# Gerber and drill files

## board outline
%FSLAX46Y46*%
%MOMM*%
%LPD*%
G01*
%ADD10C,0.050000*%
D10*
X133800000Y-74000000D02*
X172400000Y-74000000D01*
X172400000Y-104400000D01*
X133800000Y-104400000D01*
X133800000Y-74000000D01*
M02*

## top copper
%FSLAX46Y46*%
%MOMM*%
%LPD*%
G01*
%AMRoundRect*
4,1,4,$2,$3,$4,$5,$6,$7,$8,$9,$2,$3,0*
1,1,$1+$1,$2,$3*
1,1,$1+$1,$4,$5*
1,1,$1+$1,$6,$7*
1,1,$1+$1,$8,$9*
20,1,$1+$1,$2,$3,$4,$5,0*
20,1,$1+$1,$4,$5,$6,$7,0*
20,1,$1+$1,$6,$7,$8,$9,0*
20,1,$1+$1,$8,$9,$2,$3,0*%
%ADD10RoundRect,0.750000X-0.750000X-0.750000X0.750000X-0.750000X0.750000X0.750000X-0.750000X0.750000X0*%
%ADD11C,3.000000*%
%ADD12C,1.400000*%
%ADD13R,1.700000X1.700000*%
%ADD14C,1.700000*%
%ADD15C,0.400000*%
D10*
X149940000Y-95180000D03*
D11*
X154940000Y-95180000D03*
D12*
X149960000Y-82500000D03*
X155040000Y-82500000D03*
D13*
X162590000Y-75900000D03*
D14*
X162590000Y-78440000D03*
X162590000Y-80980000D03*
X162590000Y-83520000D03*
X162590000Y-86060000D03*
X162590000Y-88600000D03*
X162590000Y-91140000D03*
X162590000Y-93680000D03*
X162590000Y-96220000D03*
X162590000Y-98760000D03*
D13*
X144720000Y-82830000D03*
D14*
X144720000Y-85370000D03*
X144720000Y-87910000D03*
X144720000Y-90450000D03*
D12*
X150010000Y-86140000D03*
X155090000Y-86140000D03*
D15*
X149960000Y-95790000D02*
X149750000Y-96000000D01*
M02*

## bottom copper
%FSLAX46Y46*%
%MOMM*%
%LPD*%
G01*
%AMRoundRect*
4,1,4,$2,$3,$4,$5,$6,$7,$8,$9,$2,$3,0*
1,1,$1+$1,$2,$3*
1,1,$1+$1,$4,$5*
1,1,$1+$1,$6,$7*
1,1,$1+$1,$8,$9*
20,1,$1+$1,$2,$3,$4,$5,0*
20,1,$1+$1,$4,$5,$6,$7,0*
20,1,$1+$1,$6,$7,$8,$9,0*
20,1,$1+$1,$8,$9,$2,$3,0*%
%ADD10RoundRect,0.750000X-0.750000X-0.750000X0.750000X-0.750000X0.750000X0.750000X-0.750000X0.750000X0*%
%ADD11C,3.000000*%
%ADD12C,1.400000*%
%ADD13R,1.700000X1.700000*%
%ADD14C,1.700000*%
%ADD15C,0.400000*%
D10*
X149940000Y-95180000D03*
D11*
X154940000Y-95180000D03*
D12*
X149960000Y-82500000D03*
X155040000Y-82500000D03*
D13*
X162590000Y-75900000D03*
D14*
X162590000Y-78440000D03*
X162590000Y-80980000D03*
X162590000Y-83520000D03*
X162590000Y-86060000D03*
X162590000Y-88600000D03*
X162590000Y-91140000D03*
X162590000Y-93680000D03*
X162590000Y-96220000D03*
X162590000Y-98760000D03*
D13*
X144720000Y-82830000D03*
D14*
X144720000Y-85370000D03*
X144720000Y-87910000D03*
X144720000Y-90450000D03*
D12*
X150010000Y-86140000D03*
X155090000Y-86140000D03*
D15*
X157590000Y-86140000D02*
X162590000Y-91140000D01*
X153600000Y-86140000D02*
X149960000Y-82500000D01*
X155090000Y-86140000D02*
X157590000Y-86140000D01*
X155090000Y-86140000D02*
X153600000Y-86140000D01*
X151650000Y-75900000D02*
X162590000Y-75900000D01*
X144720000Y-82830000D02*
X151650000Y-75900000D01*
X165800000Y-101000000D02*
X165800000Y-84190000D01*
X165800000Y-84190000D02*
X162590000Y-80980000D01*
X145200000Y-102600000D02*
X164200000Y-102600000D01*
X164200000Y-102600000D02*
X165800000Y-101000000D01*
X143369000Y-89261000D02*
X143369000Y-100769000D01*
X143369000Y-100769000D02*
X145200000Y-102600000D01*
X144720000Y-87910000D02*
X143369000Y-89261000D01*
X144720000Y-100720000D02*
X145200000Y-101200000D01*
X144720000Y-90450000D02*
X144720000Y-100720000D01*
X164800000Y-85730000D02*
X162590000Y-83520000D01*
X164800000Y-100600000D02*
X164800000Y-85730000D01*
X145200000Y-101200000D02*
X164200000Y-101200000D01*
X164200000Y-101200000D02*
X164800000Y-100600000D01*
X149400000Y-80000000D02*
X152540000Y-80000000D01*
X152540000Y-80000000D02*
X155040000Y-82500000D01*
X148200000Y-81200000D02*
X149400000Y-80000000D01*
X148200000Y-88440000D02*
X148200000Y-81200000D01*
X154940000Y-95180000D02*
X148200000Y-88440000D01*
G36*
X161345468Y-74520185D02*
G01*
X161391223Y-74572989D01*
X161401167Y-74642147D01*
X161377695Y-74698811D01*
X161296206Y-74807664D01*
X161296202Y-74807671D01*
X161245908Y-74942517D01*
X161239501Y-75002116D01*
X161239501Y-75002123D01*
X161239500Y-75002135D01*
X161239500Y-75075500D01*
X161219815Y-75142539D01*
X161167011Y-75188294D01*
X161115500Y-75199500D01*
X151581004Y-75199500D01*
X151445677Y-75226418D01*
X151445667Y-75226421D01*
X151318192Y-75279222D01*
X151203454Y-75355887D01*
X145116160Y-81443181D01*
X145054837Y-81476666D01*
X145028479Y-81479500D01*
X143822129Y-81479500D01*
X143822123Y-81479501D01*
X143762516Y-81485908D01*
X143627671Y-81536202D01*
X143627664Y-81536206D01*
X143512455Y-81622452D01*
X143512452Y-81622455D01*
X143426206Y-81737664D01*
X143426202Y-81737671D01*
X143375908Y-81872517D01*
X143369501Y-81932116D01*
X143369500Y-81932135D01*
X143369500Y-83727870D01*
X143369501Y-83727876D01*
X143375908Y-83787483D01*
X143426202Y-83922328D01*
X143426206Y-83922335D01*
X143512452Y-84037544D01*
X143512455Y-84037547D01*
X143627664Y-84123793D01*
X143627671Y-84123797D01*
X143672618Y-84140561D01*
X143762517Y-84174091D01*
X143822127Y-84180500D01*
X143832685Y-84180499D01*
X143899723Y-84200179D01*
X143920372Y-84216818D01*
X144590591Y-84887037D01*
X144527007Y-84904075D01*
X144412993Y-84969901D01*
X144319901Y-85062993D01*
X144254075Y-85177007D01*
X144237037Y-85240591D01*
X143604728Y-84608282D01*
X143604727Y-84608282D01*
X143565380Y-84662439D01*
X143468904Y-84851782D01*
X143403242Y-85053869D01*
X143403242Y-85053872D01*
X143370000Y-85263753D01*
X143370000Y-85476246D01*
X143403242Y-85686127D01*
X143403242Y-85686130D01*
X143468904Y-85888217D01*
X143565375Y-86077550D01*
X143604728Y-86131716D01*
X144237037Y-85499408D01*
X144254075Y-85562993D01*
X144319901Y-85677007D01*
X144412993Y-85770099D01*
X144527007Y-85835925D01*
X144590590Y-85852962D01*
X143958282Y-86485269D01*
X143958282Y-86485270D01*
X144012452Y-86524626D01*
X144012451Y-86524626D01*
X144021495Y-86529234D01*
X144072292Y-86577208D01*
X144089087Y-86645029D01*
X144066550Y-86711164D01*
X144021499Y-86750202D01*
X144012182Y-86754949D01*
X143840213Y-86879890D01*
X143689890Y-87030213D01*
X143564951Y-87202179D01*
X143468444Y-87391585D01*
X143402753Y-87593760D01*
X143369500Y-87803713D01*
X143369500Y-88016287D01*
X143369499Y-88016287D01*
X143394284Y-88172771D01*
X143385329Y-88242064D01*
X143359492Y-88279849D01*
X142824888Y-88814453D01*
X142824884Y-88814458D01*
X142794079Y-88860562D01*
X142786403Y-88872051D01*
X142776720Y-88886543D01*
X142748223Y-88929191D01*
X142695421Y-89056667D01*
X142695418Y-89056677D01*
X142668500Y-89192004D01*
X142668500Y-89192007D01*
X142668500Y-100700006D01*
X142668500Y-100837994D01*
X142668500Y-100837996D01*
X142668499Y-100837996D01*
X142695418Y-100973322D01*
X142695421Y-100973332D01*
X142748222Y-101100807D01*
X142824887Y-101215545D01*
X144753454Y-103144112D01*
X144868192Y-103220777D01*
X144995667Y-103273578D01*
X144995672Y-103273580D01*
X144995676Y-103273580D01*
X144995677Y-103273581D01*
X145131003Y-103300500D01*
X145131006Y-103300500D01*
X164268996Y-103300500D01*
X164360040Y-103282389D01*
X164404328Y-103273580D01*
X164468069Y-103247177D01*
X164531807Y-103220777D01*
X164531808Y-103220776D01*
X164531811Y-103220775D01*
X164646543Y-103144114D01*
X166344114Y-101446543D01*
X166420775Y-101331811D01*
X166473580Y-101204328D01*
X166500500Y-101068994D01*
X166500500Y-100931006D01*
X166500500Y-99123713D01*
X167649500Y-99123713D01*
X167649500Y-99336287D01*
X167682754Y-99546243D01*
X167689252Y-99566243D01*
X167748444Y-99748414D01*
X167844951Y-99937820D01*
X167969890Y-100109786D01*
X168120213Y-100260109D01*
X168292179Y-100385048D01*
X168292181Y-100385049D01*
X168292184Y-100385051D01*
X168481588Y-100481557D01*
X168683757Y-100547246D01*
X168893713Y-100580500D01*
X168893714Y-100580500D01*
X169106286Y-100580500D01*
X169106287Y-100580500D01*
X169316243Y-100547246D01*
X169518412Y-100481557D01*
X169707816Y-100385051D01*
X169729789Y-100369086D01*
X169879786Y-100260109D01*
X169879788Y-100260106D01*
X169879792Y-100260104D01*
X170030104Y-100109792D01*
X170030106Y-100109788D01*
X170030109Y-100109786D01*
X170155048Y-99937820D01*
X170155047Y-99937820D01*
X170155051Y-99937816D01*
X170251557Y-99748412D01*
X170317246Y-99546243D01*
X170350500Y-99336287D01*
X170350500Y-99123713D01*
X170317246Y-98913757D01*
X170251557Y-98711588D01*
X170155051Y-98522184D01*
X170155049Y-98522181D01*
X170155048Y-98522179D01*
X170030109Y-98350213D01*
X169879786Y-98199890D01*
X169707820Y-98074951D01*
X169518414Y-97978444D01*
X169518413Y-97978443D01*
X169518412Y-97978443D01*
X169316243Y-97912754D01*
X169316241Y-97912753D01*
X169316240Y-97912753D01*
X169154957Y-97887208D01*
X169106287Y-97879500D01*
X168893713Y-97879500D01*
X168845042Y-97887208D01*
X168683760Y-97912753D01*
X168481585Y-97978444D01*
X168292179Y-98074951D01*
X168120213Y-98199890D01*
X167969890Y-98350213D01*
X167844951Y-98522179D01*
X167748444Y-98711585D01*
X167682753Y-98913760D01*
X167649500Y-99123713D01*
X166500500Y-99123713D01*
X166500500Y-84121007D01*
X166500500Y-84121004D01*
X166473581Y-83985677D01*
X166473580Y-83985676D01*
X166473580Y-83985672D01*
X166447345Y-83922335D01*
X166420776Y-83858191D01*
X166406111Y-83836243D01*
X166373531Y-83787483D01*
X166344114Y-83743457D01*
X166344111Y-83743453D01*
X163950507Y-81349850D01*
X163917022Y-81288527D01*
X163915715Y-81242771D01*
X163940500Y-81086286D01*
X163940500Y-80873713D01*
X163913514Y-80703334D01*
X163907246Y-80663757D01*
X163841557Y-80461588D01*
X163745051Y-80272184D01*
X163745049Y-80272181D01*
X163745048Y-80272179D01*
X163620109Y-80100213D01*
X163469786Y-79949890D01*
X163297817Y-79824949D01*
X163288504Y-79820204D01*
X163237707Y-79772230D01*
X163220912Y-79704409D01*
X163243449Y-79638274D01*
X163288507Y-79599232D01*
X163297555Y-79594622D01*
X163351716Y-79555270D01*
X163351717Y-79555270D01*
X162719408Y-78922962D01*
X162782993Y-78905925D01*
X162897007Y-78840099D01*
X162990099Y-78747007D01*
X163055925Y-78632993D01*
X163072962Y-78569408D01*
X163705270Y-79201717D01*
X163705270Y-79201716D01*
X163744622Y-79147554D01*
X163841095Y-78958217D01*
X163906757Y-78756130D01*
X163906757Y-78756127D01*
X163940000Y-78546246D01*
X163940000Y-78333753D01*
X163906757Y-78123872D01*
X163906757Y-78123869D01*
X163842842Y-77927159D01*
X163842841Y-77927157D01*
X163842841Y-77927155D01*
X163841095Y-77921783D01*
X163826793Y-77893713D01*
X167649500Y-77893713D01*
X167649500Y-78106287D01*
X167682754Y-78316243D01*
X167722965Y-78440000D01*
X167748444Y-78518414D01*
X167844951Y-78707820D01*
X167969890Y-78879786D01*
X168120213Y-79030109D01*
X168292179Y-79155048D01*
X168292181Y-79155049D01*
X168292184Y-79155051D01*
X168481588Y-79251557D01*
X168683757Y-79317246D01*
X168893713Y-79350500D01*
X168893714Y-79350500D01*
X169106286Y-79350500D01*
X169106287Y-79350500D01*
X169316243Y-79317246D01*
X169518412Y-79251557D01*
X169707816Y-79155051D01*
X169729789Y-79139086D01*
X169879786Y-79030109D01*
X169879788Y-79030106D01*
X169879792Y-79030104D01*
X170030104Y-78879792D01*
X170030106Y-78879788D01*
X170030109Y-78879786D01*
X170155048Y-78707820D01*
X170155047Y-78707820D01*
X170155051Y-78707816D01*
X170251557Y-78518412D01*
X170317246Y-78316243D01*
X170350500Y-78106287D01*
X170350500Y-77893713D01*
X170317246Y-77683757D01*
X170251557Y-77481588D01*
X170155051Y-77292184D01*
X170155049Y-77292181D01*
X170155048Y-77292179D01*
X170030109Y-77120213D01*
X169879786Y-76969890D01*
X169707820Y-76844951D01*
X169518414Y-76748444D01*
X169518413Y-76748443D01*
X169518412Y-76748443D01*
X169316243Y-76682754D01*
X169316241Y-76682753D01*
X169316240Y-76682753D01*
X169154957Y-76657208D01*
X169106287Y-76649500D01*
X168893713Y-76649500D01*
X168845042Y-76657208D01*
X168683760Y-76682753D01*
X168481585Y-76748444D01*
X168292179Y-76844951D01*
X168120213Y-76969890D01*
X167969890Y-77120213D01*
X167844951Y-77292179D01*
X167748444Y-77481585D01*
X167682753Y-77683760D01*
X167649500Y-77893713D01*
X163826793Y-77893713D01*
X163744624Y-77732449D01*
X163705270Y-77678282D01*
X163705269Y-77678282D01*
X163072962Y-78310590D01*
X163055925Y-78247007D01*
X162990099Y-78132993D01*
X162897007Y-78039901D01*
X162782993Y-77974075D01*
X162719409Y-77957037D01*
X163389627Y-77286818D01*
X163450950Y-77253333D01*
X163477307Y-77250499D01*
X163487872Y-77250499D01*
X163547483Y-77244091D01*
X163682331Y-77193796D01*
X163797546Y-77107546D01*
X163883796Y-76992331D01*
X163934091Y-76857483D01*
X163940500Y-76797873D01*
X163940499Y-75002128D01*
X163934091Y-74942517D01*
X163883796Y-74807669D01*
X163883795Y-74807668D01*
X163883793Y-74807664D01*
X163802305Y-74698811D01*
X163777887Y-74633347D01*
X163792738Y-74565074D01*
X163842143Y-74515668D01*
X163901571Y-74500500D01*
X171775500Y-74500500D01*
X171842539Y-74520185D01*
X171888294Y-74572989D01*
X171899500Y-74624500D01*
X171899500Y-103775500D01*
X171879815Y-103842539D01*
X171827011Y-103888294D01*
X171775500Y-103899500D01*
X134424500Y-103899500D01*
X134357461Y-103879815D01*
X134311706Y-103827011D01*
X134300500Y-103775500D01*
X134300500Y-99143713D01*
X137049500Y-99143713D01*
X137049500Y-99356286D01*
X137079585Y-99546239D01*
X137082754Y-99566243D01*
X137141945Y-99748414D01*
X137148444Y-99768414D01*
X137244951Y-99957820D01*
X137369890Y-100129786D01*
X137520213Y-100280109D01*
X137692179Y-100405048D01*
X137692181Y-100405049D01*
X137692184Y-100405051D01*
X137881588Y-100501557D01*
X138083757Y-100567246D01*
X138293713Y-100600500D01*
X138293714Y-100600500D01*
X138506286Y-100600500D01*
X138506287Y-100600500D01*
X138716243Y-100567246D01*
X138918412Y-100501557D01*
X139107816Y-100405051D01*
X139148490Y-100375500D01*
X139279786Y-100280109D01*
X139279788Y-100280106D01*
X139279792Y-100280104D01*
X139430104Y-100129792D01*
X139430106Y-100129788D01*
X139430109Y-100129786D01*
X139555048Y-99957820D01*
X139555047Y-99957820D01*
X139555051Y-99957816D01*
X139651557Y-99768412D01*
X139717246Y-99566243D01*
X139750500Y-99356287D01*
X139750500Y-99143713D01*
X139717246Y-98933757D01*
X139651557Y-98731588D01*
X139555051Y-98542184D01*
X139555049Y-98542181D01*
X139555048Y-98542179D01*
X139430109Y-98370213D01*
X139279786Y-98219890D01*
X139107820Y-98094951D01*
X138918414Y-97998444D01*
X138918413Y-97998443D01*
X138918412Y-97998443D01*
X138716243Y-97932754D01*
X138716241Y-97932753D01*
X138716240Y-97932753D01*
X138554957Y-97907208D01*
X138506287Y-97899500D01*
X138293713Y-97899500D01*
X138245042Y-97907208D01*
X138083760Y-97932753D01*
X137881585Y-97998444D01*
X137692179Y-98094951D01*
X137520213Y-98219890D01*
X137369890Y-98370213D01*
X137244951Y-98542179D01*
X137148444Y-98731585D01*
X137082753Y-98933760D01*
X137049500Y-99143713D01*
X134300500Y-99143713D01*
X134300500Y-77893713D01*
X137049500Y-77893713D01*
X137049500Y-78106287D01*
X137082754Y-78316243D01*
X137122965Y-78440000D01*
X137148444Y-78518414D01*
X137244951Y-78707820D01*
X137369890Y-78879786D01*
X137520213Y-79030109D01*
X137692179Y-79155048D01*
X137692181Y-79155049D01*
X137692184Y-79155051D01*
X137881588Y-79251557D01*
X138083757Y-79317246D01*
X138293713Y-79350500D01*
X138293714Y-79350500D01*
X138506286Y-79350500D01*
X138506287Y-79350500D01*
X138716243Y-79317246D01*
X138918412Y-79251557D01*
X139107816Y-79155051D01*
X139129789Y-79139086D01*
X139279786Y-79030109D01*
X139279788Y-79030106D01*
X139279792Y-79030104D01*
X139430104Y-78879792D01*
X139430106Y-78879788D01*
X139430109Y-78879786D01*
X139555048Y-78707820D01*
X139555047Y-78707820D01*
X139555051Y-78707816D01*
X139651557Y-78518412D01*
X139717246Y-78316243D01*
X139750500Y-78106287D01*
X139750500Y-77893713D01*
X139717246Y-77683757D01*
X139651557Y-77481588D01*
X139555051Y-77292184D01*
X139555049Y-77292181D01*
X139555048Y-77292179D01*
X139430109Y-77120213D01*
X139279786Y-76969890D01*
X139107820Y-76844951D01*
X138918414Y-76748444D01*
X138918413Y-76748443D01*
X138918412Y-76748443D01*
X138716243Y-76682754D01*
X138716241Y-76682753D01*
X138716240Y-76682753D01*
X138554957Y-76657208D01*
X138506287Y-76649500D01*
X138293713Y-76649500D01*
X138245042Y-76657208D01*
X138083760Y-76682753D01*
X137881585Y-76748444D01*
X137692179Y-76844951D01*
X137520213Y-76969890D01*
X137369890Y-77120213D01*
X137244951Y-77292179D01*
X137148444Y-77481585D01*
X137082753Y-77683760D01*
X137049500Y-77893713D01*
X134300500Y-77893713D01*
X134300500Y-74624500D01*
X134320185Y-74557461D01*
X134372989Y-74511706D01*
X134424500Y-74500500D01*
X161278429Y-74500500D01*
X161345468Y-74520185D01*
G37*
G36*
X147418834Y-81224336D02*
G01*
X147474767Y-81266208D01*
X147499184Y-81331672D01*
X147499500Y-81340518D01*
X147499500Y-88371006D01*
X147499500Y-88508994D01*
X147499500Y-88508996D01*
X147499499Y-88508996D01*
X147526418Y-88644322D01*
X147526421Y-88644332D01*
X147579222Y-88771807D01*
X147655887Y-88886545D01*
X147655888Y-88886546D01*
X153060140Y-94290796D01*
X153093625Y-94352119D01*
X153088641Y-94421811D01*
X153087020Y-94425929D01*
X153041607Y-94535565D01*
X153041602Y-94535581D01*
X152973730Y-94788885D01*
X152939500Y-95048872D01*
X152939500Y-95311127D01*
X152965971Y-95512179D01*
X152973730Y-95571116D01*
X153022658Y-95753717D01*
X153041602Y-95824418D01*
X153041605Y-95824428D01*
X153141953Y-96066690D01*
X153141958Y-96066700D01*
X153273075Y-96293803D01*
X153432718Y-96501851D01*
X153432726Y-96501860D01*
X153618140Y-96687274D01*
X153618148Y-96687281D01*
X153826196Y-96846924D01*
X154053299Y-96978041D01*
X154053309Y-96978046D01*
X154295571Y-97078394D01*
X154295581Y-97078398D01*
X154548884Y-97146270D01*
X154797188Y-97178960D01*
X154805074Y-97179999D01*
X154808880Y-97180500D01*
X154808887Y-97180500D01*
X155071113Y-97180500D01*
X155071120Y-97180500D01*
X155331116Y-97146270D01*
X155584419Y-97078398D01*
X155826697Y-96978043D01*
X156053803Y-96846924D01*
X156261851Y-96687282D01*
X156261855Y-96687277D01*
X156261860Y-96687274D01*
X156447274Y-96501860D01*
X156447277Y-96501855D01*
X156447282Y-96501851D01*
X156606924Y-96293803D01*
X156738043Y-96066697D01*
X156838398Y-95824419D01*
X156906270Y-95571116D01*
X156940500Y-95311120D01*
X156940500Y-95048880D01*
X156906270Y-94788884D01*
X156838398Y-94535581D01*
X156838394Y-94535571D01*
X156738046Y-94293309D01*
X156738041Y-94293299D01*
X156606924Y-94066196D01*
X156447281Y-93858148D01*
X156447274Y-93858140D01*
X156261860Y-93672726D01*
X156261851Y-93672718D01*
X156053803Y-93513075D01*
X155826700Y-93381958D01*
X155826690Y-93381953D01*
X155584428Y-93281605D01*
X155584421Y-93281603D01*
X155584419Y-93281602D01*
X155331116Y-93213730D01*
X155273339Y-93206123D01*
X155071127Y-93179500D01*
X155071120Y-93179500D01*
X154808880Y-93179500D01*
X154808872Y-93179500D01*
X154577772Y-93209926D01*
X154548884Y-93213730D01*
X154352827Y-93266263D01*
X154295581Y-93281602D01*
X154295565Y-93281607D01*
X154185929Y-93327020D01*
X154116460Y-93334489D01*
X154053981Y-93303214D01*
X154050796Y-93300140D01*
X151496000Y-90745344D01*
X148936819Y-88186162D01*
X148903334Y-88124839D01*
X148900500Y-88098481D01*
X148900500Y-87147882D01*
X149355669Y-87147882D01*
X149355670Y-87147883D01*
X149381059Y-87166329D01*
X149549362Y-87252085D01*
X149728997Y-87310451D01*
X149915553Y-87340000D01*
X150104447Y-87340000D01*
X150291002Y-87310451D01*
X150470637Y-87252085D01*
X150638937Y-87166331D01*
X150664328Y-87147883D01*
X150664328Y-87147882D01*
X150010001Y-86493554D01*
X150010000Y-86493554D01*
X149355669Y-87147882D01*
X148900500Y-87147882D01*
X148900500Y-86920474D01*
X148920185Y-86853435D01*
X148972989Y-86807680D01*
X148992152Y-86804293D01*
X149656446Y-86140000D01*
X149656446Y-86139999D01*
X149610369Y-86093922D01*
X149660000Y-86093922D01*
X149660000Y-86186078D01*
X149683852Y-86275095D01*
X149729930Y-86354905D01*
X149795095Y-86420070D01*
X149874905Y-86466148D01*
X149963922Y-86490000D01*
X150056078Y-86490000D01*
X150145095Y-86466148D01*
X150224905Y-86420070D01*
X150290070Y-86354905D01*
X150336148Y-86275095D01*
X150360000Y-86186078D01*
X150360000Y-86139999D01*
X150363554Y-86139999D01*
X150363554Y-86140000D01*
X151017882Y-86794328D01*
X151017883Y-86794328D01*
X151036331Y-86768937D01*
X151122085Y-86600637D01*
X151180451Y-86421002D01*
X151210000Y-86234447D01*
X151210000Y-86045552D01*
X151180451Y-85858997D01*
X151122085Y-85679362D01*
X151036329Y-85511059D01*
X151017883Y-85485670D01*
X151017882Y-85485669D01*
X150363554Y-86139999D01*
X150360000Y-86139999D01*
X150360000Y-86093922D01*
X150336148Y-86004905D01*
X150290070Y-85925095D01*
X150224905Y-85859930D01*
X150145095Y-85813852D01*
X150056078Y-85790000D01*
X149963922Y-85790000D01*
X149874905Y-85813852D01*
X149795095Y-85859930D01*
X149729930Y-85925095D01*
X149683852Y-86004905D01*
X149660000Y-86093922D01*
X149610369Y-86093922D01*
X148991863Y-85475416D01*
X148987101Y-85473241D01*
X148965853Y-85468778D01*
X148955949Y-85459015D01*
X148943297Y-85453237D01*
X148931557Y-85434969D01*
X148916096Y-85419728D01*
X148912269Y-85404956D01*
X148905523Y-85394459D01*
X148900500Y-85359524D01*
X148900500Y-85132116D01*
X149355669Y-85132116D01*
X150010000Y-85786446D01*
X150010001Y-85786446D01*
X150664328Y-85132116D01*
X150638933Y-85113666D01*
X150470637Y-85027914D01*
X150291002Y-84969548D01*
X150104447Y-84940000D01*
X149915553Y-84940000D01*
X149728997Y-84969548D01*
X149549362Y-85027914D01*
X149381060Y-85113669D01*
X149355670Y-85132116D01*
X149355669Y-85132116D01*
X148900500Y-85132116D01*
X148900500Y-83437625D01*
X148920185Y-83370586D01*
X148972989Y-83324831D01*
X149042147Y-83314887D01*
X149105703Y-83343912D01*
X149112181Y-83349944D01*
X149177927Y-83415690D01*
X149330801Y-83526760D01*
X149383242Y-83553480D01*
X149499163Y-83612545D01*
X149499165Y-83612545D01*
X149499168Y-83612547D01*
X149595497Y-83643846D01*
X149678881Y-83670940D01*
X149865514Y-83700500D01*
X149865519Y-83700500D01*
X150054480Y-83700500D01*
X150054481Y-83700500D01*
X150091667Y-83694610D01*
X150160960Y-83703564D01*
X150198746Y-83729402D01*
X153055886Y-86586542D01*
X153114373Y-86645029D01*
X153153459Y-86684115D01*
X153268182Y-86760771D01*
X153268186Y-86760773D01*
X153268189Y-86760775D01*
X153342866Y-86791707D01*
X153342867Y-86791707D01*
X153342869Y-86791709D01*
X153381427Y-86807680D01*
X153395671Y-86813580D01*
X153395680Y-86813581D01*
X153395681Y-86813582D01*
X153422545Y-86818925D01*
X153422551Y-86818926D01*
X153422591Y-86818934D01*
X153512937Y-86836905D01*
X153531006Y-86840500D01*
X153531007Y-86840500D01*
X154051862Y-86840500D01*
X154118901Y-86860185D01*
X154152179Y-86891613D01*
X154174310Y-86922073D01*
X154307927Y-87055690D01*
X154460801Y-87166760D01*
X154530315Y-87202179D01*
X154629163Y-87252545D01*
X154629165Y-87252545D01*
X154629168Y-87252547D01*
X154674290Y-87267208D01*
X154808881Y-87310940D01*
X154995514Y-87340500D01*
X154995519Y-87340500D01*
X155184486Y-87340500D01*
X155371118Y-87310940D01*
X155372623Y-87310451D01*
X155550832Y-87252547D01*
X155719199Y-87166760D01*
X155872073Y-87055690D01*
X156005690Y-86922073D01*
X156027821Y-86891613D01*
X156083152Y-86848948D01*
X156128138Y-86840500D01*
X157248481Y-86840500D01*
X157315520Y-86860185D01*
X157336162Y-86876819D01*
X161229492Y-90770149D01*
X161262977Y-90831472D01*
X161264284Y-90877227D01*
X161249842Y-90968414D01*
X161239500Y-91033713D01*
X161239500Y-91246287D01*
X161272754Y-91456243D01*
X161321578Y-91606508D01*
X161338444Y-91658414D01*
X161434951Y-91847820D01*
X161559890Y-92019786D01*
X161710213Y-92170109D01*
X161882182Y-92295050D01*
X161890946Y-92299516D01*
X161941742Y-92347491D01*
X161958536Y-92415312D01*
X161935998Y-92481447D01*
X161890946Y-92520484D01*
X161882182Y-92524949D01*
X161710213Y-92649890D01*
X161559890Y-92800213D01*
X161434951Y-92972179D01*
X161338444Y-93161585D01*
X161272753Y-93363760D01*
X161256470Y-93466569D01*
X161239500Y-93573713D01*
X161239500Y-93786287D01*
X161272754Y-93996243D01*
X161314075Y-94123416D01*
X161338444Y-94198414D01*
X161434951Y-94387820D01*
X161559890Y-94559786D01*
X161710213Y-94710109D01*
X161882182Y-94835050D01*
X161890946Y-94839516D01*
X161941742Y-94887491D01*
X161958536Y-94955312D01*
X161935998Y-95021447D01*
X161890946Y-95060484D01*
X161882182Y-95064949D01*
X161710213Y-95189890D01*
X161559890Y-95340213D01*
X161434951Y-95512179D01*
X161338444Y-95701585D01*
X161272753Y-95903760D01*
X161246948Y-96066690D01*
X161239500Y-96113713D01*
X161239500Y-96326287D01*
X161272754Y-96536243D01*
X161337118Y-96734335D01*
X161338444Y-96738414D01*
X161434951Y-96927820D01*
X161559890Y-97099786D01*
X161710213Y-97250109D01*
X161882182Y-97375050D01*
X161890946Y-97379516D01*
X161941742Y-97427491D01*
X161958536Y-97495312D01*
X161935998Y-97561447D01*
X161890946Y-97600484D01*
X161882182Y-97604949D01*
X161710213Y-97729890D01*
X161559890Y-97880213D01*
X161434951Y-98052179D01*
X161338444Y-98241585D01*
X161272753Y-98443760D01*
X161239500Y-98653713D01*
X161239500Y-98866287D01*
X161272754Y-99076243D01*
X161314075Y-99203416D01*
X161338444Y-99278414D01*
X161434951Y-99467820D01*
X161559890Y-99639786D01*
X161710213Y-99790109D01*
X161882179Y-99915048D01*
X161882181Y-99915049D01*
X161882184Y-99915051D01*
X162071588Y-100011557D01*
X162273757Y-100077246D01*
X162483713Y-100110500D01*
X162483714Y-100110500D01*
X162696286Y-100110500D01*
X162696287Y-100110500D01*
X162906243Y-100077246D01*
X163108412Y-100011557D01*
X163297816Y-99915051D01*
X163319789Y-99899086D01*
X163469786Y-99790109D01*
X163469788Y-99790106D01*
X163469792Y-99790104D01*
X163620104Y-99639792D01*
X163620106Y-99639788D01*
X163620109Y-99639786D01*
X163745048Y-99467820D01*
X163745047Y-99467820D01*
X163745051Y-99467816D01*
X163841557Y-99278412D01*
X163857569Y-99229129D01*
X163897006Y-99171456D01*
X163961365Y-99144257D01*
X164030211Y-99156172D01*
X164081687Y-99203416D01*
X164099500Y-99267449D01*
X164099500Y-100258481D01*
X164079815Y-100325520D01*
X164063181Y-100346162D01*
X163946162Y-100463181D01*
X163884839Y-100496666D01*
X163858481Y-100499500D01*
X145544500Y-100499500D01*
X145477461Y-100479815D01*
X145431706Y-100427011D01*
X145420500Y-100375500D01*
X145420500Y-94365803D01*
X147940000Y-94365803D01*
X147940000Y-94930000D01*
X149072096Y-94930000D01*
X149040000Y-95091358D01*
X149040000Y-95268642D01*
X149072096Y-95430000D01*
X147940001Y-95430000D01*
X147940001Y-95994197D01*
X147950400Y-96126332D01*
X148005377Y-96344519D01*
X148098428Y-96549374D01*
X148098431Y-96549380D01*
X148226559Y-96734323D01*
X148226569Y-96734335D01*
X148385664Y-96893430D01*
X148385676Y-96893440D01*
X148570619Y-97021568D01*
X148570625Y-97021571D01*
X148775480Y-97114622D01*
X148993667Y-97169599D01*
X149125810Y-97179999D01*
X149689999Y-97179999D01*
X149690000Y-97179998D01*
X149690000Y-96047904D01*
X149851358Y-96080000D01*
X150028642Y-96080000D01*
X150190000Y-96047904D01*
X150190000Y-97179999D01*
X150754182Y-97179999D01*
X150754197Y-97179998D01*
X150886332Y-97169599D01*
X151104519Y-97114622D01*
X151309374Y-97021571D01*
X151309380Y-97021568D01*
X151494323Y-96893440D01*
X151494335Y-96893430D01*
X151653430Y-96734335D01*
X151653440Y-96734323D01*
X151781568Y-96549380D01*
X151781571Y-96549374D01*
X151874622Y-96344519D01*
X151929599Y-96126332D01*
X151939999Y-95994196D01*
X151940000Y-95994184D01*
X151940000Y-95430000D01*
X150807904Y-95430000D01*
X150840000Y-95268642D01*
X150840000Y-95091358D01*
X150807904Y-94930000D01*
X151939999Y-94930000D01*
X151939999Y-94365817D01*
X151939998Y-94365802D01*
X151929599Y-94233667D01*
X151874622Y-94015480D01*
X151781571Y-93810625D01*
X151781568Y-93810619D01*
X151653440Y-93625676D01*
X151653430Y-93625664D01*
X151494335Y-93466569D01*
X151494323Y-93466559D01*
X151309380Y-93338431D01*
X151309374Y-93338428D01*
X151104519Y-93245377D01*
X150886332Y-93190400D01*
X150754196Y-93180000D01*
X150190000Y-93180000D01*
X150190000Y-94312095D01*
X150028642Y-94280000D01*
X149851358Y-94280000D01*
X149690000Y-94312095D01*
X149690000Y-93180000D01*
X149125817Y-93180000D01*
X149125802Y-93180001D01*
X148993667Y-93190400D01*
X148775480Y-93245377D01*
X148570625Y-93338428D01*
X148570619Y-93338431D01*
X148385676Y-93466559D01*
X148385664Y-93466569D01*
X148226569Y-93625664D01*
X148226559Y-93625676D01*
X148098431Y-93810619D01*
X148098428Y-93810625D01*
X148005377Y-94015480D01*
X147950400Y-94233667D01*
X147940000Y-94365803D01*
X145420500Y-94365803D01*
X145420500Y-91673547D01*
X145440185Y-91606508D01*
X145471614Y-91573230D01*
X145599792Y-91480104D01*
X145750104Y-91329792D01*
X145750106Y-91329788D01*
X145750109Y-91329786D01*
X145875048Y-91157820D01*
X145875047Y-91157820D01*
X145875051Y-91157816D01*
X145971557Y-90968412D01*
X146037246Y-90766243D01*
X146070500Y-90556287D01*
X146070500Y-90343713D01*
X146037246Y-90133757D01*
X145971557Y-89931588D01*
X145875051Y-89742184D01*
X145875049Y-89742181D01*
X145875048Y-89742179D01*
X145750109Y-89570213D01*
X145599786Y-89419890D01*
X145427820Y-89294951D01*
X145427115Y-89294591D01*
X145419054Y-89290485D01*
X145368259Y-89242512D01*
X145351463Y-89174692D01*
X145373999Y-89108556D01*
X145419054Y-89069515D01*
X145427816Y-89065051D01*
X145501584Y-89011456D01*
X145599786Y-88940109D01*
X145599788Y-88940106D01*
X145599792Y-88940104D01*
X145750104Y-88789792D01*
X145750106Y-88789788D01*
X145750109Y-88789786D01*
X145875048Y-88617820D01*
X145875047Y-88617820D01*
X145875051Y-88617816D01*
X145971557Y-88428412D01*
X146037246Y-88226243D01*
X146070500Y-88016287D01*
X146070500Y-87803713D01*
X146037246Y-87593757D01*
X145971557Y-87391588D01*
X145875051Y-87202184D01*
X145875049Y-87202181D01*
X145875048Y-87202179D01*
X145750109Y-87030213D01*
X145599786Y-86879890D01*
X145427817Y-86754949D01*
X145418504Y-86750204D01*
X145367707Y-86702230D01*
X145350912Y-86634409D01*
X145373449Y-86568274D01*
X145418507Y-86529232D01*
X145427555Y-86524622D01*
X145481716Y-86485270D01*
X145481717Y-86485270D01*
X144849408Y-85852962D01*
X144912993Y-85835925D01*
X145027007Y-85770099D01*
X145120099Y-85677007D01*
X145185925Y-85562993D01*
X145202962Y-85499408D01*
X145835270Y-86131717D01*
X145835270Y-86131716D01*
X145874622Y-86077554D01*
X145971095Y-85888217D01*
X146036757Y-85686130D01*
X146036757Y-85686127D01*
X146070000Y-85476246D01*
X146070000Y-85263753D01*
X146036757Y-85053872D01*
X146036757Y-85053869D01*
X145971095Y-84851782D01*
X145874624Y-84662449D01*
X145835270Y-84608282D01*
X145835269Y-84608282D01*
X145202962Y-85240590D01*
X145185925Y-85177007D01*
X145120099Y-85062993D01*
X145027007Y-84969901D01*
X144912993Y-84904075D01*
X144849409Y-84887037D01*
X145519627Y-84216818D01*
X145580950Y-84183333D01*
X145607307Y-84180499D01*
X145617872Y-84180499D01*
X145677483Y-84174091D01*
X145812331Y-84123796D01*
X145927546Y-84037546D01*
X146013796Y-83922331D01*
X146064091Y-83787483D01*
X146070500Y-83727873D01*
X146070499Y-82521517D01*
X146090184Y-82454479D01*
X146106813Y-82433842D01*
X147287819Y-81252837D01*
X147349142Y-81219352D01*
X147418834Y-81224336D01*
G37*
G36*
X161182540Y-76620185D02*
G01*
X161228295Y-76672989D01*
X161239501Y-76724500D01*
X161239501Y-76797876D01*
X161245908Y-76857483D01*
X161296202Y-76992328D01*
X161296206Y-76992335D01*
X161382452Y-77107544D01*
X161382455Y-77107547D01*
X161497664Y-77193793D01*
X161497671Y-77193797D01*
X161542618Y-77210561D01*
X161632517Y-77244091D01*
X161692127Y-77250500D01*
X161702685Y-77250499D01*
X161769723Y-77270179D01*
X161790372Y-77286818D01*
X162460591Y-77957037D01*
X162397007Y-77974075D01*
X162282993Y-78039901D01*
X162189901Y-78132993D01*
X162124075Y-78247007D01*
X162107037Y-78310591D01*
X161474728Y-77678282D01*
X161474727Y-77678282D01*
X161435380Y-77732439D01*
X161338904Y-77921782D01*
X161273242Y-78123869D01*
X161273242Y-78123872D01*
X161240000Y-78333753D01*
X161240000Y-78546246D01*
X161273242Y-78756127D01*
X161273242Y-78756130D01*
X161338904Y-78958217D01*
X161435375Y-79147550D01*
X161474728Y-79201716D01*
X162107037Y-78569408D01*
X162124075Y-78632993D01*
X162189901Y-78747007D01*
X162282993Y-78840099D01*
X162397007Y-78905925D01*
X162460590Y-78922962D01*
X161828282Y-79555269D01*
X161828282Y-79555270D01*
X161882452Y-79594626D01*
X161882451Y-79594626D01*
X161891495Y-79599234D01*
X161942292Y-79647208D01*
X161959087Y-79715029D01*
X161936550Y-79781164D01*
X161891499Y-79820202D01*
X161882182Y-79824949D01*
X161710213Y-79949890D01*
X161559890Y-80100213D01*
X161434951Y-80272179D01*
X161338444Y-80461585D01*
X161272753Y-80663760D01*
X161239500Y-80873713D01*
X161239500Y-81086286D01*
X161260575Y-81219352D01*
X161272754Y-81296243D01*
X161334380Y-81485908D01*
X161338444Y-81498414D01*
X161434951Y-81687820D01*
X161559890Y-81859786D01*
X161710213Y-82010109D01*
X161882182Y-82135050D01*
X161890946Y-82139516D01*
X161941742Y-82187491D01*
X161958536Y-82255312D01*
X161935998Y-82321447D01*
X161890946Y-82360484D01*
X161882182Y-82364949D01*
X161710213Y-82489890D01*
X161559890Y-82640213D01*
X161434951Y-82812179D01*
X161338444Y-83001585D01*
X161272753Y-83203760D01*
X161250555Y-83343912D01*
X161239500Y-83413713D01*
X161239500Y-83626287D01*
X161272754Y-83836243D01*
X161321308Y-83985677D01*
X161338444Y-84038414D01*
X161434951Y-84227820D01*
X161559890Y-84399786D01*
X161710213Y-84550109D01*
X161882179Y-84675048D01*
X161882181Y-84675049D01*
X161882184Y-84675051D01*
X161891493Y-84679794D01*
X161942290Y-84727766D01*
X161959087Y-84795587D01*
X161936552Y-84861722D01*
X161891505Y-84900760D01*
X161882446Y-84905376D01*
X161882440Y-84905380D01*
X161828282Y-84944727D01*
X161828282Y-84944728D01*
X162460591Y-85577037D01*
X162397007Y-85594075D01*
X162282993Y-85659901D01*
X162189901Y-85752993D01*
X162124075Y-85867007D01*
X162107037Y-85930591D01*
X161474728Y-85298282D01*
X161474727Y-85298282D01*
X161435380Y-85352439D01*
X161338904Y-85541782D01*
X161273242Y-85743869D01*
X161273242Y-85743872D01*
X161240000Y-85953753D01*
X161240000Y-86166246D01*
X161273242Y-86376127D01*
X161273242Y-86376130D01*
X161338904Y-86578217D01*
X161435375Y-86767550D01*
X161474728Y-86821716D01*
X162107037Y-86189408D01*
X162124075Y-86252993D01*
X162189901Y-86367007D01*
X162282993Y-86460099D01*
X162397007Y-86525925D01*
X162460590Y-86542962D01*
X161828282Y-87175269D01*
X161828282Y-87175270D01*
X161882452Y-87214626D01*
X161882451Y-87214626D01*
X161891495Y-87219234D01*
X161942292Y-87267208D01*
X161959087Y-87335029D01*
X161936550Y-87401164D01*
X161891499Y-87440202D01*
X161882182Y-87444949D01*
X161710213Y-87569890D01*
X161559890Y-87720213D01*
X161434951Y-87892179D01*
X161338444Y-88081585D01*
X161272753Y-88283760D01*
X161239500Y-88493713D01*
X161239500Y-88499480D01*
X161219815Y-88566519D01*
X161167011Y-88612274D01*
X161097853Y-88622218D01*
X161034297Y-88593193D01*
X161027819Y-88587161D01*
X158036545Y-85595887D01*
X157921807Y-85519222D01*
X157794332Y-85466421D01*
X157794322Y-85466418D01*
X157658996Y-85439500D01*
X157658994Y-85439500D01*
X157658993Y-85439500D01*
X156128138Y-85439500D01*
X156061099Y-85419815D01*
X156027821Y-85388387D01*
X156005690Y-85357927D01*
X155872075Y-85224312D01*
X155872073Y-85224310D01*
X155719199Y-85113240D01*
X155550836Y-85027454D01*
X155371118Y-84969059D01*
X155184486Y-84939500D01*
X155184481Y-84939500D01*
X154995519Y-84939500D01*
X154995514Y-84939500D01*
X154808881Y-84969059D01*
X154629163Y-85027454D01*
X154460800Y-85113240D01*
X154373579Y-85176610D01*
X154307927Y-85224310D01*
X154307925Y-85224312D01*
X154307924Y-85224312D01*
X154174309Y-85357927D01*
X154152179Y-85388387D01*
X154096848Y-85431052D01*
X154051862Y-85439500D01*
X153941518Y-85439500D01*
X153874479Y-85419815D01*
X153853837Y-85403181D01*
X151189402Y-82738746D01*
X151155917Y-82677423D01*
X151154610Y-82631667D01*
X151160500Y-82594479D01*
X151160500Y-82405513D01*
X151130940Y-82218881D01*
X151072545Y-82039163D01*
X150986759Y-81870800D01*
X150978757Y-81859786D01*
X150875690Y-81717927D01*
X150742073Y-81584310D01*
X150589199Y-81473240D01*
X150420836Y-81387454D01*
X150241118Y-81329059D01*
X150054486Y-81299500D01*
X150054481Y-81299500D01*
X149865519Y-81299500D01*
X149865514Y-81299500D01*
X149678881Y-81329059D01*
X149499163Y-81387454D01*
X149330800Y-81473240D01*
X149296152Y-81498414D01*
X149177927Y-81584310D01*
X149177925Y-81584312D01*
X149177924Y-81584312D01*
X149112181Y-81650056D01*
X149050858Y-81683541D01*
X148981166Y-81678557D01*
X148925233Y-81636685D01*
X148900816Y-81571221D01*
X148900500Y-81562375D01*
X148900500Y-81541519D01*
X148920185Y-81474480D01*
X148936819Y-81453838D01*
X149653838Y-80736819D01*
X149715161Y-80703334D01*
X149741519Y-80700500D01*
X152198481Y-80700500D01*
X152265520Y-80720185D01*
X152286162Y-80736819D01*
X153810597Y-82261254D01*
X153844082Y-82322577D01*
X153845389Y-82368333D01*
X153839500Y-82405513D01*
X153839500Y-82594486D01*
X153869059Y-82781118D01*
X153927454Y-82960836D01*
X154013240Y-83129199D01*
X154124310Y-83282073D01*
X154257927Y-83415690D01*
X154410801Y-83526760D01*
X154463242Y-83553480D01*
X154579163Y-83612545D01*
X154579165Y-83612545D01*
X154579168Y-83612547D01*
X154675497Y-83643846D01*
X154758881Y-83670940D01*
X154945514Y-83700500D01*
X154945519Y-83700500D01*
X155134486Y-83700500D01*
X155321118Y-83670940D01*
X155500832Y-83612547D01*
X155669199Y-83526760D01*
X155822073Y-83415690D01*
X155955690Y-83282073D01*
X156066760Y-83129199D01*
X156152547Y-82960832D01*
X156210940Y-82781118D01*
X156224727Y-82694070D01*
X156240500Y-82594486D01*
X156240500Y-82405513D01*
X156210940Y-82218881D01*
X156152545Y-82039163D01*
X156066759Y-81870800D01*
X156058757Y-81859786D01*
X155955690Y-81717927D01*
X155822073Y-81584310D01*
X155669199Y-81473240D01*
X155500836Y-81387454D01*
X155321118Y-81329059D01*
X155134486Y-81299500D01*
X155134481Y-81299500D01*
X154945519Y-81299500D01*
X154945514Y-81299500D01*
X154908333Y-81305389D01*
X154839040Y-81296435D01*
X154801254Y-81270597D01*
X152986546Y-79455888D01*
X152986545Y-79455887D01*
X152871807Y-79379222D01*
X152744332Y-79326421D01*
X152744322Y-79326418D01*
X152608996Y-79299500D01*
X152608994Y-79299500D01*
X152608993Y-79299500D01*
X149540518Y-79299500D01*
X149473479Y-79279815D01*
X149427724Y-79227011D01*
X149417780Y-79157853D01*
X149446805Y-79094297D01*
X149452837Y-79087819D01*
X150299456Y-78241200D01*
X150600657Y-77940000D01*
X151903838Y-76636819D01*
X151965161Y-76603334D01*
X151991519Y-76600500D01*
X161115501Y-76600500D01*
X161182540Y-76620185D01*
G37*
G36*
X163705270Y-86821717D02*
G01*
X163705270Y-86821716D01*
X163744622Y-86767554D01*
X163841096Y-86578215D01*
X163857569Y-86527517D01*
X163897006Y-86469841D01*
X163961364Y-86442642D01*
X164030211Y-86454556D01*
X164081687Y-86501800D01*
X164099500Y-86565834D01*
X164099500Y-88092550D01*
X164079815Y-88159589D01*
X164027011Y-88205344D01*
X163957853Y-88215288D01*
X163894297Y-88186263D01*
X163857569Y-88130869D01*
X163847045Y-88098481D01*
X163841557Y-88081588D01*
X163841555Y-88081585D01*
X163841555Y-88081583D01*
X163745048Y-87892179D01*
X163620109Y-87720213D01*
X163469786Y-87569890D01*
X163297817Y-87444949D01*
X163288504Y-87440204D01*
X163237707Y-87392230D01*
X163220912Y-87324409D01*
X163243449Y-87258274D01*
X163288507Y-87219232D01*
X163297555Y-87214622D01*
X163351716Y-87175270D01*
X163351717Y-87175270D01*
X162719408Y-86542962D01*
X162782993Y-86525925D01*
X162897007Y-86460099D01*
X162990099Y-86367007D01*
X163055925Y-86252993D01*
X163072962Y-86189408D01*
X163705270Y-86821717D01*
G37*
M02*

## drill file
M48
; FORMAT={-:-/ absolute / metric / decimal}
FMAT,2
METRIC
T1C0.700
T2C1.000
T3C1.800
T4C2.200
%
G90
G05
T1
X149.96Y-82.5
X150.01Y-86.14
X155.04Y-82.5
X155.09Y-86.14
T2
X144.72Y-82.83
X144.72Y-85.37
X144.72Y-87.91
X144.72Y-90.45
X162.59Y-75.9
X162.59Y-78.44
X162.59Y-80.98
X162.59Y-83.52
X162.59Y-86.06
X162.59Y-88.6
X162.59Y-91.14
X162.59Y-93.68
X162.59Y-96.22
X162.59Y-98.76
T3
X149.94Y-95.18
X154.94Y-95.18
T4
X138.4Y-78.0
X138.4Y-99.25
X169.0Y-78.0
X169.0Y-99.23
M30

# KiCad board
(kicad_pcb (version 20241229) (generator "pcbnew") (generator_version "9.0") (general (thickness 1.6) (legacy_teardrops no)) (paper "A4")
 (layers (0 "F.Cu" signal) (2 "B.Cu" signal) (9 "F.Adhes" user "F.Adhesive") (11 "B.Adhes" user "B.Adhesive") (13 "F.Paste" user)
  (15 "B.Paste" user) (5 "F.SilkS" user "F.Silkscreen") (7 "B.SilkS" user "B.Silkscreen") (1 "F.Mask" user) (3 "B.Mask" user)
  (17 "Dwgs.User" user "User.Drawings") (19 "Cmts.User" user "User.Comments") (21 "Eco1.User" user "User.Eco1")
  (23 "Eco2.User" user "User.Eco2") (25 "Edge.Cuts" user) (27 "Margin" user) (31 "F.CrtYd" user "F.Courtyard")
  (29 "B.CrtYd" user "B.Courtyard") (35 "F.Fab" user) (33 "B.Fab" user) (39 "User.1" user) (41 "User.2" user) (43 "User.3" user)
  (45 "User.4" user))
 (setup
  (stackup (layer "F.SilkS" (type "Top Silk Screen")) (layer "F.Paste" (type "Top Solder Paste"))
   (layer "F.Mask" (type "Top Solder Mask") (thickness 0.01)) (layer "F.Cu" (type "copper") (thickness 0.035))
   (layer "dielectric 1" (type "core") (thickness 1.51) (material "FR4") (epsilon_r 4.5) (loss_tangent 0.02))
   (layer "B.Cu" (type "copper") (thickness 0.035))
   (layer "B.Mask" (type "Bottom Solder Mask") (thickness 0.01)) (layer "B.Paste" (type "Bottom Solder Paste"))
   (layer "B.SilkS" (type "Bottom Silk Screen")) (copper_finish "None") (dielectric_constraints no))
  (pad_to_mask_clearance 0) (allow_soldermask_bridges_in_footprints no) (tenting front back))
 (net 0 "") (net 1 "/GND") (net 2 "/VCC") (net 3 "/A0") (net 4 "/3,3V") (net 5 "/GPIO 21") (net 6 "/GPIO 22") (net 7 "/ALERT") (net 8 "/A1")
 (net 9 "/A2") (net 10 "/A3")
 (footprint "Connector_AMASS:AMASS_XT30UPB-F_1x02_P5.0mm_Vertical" (layer "F.Cu") (at 149.94 95.18)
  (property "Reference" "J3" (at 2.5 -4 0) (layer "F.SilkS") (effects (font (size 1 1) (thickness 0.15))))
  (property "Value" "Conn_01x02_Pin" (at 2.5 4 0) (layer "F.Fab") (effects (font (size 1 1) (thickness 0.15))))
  (pad "1" thru_hole roundrect (at 0 0) (size 3 3) (drill 1.8) (layers "*.Cu" "*.Mask") (remove_unused_layers no) (roundrect_rratio 0.25)
   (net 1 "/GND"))
  (pad "2" thru_hole circle (at 5 0) (size 3 3) (drill 1.8) (layers "*.Cu" "*.Mask") (remove_unused_layers no) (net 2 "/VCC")))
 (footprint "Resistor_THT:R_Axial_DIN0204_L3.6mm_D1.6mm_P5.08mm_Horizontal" (layer "F.Cu") (at 149.96 82.5)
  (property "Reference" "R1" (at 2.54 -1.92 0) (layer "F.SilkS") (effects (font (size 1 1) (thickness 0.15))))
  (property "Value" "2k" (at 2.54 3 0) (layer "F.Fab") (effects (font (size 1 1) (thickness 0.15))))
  (pad "1" thru_hole circle (at 0 0) (size 1.4 1.4) (drill 0.7) (layers "*.Cu" "*.Mask") (remove_unused_layers no) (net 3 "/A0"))
  (pad "2" thru_hole circle (at 5.08 0) (size 1.4 1.4) (drill 0.7) (layers "*.Cu" "*.Mask") (remove_unused_layers no) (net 2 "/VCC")))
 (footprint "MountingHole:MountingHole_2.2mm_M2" (layer "F.Cu") (at 169 78)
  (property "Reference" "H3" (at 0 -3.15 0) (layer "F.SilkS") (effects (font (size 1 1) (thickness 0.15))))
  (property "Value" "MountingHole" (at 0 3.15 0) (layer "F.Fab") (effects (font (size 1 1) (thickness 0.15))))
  (pad "" np_thru_hole circle (at 0 0) (size 2.2 2.2) (drill 2.2) (layers "*.Cu" "*.Mask")))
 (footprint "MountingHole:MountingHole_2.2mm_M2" (layer "F.Cu") (at 169 99.23)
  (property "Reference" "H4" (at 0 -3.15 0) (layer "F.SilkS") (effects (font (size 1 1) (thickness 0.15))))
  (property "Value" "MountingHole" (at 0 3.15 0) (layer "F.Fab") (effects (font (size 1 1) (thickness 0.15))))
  (pad "" np_thru_hole circle (at 0 0) (size 2.2 2.2) (drill 2.2) (layers "*.Cu" "*.Mask")))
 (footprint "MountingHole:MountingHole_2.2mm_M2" (layer "F.Cu") (at 138.4 78)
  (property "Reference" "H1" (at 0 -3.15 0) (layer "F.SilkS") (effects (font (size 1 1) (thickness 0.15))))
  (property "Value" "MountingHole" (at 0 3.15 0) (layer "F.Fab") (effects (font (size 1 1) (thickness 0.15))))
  (pad "" np_thru_hole circle (at 0 0) (size 2.2 2.2) (drill 2.2) (layers "*.Cu" "*.Mask")))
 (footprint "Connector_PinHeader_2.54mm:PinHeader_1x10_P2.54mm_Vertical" (layer "F.Cu") (at 162.59 75.9)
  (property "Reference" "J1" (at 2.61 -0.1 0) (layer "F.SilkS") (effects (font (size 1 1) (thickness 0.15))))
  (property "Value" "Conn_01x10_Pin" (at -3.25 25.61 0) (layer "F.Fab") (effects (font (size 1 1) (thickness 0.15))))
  (pad "1" thru_hole rect (at 0 0) (size 1.7 1.7) (drill 1) (layers "*.Cu" "*.Mask") (remove_unused_layers no) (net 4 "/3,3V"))
  (pad "2" thru_hole circle (at 0 2.54) (size 1.7 1.7) (drill 1) (layers "*.Cu" "*.Mask") (remove_unused_layers no) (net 1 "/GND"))
  (pad "3" thru_hole circle (at 0 5.08) (size 1.7 1.7) (drill 1) (layers "*.Cu" "*.Mask") (remove_unused_layers no) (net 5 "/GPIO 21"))
  (pad "4" thru_hole circle (at 0 7.62) (size 1.7 1.7) (drill 1) (layers "*.Cu" "*.Mask") (remove_unused_layers no) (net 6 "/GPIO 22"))
  (pad "5" thru_hole circle (at 0 10.16) (size 1.7 1.7) (drill 1) (layers "*.Cu" "*.Mask") (remove_unused_layers no) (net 1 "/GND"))
  (pad "6" thru_hole circle (at 0 12.7) (size 1.7 1.7) (drill 1) (layers "*.Cu" "*.Mask") (remove_unused_layers no) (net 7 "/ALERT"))
  (pad "7" thru_hole circle (at 0 15.24) (size 1.7 1.7) (drill 1) (layers "*.Cu" "*.Mask") (remove_unused_layers no) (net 3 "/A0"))
  (pad "8" thru_hole circle (at 0 17.78) (size 1.7 1.7) (drill 1) (layers "*.Cu" "*.Mask") (remove_unused_layers no) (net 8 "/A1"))
  (pad "9" thru_hole circle (at 0 20.32) (size 1.7 1.7) (drill 1) (layers "*.Cu" "*.Mask") (remove_unused_layers no) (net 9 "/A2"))
  (pad "10" thru_hole circle (at 0 22.86) (size 1.7 1.7) (drill 1) (layers "*.Cu" "*.Mask") (remove_unused_layers no) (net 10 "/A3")))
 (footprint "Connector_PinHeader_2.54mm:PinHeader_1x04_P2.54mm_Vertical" (layer "F.Cu") (at 144.72 82.83)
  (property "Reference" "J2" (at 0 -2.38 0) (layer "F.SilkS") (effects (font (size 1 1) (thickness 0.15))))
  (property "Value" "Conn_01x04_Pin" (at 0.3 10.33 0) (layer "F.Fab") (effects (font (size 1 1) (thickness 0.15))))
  (pad "1" thru_hole rect (at 0 0) (size 1.7 1.7) (drill 1) (layers "*.Cu" "*.Mask") (remove_unused_layers no) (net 4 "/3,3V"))
  (pad "2" thru_hole circle (at 0 2.54) (size 1.7 1.7) (drill 1) (layers "*.Cu" "*.Mask") (remove_unused_layers no) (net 1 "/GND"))
  (pad "3" thru_hole circle (at 0 5.08) (size 1.7 1.7) (drill 1) (layers "*.Cu" "*.Mask") (remove_unused_layers no) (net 5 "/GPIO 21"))
  (pad "4" thru_hole circle (at 0 7.62) (size 1.7 1.7) (drill 1) (layers "*.Cu" "*.Mask") (remove_unused_layers no) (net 6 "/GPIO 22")))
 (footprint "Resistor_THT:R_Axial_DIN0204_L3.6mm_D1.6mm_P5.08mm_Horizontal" (layer "F.Cu") (at 150.01 86.14)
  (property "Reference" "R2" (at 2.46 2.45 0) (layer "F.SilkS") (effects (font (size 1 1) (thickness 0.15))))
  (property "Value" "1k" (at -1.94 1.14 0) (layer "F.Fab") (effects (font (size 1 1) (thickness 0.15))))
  (pad "1" thru_hole circle (at 0 0) (size 1.4 1.4) (drill 0.7) (layers "*.Cu" "*.Mask") (remove_unused_layers no) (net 1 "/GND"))
  (pad "2" thru_hole circle (at 5.08 0) (size 1.4 1.4) (drill 0.7) (layers "*.Cu" "*.Mask") (remove_unused_layers no) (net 3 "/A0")))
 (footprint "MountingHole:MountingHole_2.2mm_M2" (layer "F.Cu") (at 138.4 99.25)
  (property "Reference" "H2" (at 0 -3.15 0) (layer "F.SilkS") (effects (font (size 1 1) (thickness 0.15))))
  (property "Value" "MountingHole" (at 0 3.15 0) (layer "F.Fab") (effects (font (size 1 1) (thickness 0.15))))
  (pad "" np_thru_hole circle (at 0 0) (size 2.2 2.2) (drill 2.2) (layers "*.Cu" "*.Mask")))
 (gr_rect (start 133.8 74) (end 172.4 104.4) (stroke (width 0.05) (type default)) (fill no) (layer "Edge.Cuts"))
 (segment (start 157.59 86.14) (end 162.59 91.14) (width 0.4) (layer "B.Cu") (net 3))
 (segment (start 153.6 86.14) (end 149.96 82.5) (width 0.4) (layer "B.Cu") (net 3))
 (segment (start 155.09 86.14) (end 157.59 86.14) (width 0.4) (layer "B.Cu") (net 3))
 (segment (start 155.09 86.14) (end 153.6 86.14) (width 0.4) (layer "B.Cu") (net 3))
 (segment (start 149.96 95.79) (end 149.75 96) (width 0.4) (layer "F.Cu") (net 1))
 (segment (start 151.65 75.9) (end 162.59 75.9) (width 0.4) (layer "B.Cu") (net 4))
 (segment (start 144.72 82.83) (end 151.65 75.9) (width 0.4) (layer "B.Cu") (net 4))
 (segment (start 165.8 101) (end 165.8 84.19) (width 0.4) (layer "B.Cu") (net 5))
 (segment (start 165.8 84.19) (end 162.59 80.98) (width 0.4) (layer "B.Cu") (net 5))
 (segment (start 145.2 102.6) (end 164.2 102.6) (width 0.4) (layer "B.Cu") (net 5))
 (segment (start 164.2 102.6) (end 165.8 101) (width 0.4) (layer "B.Cu") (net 5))
 (segment (start 143.369 89.261) (end 143.369 100.769) (width 0.4) (layer "B.Cu") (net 5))
 (segment (start 143.369 100.769) (end 145.2 102.6) (width 0.4) (layer "B.Cu") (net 5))
 (segment (start 144.72 87.91) (end 143.369 89.261) (width 0.4) (layer "B.Cu") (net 5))
 (segment (start 144.72 100.72) (end 145.2 101.2) (width 0.4) (layer "B.Cu") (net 6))
 (segment (start 144.72 90.45) (end 144.72 100.72) (width 0.4) (layer "B.Cu") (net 6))
 (segment (start 164.8 85.73) (end 162.59 83.52) (width 0.4) (layer "B.Cu") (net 6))
 (segment (start 164.8 100.6) (end 164.8 85.73) (width 0.4) (layer "B.Cu") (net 6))
 (segment (start 145.2 101.2) (end 164.2 101.2) (width 0.4) (layer "B.Cu") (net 6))
 (segment (start 164.2 101.2) (end 164.8 100.6) (width 0.4) (layer "B.Cu") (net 6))
 (segment (start 149.4 80) (end 152.54 80) (width 0.4) (layer "B.Cu") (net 2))
 (segment (start 152.54 80) (end 155.04 82.5) (width 0.4) (layer "B.Cu") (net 2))
 (segment (start 148.2 81.2) (end 149.4 80) (width 0.4) (layer "B.Cu") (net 2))
 (segment (start 148.2 88.44) (end 148.2 81.2) (width 0.4) (layer "B.Cu") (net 2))
 (segment (start 154.94 95.18) (end 148.2 88.44) (width 0.4) (layer "B.Cu") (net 2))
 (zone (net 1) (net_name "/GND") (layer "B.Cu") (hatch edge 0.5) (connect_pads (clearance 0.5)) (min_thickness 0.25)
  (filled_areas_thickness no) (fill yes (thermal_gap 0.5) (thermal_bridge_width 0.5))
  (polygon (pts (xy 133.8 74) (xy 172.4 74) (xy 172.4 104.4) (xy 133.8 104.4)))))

